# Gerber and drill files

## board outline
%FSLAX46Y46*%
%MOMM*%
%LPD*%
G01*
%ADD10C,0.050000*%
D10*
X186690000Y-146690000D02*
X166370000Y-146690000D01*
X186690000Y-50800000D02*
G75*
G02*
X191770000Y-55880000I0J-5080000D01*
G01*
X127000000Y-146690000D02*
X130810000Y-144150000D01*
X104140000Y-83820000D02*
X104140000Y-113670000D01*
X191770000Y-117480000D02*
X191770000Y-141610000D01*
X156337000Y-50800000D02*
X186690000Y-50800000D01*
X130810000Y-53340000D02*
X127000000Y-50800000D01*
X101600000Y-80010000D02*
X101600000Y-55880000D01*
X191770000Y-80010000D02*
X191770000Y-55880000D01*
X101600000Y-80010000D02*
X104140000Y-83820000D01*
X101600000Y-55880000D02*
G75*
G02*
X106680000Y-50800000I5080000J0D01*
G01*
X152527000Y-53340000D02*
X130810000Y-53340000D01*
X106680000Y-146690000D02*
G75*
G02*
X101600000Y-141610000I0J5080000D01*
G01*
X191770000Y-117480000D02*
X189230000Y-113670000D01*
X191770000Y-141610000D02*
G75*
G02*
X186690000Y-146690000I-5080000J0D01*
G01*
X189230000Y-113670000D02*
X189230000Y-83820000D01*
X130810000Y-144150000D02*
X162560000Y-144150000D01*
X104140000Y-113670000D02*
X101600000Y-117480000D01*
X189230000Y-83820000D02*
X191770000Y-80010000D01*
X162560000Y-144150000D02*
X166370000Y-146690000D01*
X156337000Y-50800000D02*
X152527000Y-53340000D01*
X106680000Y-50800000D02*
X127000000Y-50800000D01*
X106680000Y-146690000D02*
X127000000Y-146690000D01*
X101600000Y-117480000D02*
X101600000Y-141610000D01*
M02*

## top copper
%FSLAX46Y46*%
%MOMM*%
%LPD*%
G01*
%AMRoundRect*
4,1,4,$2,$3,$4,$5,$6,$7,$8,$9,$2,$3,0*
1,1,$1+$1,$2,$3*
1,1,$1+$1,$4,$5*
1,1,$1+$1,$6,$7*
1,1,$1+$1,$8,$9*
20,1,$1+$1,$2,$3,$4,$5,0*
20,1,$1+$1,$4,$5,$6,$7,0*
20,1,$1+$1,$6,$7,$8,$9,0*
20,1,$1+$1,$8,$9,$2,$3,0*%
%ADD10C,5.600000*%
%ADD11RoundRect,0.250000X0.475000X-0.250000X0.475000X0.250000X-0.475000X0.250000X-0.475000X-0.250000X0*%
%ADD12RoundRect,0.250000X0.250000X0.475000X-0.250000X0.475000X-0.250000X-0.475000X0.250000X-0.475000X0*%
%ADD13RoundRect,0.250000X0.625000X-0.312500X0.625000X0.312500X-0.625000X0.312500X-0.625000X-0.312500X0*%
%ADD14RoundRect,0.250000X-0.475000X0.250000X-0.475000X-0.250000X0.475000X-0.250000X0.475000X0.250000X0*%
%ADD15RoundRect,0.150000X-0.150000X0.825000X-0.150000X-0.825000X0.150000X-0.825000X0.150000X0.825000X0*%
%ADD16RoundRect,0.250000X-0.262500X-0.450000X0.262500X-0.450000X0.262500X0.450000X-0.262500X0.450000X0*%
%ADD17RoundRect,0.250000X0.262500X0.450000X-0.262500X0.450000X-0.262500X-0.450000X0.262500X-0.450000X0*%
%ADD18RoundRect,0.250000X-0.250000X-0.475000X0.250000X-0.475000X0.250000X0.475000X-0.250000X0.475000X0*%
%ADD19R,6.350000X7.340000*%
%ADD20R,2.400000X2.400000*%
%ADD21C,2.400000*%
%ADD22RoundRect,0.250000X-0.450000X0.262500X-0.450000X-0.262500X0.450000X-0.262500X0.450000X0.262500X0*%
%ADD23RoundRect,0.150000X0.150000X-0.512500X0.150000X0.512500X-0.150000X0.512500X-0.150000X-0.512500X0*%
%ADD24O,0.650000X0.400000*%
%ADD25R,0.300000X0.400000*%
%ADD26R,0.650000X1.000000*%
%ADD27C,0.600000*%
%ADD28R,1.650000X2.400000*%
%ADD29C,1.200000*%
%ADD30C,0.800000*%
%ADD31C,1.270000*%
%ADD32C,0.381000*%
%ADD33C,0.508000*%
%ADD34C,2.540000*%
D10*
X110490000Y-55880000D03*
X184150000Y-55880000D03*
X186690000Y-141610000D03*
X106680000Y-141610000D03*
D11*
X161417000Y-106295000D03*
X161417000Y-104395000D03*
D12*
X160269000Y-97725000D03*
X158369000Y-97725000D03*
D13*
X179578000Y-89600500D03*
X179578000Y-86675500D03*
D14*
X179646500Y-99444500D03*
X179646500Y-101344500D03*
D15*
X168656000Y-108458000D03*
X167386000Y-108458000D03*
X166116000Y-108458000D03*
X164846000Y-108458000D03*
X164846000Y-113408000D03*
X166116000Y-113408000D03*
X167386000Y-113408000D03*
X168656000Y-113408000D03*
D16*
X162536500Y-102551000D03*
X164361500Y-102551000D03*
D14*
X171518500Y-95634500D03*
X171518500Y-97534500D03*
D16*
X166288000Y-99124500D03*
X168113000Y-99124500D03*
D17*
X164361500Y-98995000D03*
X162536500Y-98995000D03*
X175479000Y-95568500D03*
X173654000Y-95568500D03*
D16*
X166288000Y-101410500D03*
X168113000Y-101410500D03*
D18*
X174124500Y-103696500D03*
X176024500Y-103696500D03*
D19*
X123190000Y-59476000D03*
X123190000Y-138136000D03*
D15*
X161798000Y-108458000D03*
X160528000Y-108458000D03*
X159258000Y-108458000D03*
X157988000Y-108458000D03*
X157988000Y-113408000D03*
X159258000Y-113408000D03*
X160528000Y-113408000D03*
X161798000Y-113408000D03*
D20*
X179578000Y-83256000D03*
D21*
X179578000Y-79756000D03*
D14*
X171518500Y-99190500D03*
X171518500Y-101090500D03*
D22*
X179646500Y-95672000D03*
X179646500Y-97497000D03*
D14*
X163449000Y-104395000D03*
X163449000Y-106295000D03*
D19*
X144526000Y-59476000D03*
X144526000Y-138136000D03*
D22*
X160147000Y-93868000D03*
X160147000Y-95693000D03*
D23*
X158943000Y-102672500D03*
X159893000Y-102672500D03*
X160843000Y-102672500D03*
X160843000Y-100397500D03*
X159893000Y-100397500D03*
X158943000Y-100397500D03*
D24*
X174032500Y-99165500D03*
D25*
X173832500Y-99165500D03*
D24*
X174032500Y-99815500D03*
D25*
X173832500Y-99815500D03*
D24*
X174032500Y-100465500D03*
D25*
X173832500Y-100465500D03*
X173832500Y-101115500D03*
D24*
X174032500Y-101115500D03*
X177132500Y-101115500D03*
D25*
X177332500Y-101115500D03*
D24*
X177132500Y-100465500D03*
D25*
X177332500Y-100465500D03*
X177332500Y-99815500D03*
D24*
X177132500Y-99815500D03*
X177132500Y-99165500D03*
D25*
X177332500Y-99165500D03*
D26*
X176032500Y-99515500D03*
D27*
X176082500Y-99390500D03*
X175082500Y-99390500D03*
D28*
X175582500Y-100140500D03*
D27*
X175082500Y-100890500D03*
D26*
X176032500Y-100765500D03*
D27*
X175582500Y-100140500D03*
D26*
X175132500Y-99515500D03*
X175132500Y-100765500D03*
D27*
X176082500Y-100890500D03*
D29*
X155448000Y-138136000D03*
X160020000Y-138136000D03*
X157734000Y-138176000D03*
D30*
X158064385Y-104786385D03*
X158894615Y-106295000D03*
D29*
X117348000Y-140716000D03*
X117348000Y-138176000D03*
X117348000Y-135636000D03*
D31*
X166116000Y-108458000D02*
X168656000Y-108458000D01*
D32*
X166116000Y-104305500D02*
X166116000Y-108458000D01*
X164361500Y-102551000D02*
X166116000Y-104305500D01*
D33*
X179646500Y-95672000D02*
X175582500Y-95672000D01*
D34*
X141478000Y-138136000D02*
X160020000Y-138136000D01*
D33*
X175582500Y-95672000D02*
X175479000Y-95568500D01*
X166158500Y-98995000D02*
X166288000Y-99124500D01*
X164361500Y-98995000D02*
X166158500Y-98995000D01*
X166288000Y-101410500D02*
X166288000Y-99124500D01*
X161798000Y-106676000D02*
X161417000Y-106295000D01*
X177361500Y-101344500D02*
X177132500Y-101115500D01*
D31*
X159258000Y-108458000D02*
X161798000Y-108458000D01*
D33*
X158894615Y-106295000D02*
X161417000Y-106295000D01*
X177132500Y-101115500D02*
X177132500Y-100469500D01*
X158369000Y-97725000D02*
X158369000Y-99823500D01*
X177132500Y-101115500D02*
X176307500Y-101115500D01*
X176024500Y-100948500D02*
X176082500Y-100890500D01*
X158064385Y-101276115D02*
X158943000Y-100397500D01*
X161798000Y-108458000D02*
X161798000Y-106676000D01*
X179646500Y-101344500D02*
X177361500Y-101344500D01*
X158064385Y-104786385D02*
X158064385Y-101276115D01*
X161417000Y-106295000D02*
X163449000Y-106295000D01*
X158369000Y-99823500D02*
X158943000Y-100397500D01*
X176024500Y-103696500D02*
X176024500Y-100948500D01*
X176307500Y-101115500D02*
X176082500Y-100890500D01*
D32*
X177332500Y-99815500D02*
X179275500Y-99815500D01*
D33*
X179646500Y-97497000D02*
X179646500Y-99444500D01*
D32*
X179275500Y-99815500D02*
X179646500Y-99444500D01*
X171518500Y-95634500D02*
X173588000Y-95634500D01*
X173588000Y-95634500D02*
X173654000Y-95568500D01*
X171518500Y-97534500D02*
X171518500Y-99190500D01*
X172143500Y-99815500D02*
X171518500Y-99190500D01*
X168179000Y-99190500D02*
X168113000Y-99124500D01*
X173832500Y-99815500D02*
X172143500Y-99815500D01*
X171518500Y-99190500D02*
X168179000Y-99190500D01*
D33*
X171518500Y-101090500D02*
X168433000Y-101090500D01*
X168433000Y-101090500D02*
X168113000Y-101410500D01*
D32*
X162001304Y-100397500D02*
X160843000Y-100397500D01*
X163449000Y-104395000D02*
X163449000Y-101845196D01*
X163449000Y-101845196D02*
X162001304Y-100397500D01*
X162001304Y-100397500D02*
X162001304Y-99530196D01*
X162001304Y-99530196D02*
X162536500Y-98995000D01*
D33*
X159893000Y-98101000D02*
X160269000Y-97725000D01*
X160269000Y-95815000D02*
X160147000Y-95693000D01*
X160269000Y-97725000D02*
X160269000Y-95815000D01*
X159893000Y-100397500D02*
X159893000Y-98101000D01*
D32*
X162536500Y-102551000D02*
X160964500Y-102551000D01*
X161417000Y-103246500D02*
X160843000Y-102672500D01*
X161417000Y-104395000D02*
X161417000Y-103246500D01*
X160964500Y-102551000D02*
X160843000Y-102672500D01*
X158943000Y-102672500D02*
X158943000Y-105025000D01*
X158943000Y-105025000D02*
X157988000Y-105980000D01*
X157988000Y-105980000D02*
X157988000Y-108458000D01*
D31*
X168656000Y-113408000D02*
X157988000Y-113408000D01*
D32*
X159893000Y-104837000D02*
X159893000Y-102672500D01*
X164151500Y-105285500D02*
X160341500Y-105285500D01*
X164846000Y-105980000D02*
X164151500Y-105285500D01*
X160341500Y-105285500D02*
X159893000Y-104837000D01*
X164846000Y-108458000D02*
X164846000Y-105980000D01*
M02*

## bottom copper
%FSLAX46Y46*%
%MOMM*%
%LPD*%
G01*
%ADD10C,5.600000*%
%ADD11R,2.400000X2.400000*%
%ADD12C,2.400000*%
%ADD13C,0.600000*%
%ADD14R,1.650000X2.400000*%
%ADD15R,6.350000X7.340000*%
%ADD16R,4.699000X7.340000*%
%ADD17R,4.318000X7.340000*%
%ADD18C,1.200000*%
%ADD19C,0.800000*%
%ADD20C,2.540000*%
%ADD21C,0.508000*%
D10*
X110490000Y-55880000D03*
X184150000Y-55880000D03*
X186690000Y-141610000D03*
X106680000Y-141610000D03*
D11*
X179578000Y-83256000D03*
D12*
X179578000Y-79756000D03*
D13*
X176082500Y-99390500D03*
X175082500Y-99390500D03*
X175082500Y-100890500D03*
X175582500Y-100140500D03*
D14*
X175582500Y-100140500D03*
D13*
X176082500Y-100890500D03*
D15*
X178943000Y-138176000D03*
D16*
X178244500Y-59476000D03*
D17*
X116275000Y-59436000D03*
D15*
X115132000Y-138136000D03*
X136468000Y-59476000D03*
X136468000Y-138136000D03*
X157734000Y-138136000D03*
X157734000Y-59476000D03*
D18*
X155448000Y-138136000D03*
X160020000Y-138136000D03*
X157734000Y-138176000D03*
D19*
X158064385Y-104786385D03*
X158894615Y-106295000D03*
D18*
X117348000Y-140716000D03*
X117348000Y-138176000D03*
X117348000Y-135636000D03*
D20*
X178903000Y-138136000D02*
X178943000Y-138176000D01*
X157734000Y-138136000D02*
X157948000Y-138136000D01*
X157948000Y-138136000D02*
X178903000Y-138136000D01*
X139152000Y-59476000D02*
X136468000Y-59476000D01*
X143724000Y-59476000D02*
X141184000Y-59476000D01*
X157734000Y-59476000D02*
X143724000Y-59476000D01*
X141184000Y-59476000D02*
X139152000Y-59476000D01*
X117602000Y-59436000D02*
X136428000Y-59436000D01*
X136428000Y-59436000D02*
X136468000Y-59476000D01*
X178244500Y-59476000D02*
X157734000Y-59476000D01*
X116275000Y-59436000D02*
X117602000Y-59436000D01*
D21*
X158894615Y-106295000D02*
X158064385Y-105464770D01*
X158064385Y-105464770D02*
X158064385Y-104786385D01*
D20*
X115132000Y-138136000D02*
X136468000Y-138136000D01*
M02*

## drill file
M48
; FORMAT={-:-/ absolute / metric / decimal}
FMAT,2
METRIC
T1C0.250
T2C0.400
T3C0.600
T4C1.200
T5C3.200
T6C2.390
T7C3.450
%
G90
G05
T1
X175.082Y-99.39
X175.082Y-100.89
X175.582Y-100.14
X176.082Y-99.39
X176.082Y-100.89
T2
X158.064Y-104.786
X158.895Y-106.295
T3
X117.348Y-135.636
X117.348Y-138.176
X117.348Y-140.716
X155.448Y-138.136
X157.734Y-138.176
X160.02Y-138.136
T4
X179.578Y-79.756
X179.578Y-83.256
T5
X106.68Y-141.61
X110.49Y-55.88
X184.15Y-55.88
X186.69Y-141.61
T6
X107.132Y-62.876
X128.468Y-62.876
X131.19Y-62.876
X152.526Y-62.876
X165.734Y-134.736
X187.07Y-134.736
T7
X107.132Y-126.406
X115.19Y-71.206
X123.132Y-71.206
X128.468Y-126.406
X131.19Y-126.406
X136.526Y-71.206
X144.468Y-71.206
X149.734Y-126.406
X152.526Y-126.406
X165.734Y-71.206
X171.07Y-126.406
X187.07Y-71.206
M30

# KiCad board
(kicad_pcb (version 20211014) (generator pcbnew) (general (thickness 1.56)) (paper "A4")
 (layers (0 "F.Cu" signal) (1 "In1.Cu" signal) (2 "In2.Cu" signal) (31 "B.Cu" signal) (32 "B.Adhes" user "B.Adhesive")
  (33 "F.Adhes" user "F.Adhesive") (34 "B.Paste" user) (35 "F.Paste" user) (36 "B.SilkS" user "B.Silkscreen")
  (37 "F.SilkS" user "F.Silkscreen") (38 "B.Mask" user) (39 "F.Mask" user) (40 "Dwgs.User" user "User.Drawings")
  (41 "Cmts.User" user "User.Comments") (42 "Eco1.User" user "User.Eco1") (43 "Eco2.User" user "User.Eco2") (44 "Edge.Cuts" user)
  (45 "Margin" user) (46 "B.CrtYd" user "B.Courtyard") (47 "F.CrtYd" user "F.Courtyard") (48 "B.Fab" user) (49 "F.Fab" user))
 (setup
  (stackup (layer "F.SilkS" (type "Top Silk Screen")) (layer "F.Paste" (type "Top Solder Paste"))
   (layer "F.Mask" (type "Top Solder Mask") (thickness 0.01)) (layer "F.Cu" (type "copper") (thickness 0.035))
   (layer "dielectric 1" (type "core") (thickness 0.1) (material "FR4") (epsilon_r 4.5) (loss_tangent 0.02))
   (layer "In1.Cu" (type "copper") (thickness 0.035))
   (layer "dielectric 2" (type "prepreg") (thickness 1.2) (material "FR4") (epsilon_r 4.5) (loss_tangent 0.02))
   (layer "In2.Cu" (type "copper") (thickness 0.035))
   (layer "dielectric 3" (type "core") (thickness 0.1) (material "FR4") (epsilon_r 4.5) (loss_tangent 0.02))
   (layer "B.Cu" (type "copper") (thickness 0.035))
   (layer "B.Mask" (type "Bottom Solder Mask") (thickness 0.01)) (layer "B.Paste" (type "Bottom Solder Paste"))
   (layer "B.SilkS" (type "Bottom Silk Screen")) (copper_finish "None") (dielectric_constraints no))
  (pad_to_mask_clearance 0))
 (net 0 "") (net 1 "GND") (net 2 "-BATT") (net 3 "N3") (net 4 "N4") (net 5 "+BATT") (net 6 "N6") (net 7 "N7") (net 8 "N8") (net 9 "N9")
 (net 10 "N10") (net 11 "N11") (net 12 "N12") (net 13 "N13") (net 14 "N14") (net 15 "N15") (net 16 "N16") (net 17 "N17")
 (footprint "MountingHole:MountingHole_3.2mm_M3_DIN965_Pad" (layer "F.Cu") (at 110.49 55.88)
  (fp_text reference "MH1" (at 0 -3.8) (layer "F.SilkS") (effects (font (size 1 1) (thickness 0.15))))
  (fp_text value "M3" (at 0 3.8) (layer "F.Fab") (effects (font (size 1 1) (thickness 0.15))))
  (pad "1" thru_hole circle (at 0 0) (size 5.6 5.6) (drill 3.2) (layers *.Cu *.Mask) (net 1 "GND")))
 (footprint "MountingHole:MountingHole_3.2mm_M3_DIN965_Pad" (layer "F.Cu") (at 184.15 55.88)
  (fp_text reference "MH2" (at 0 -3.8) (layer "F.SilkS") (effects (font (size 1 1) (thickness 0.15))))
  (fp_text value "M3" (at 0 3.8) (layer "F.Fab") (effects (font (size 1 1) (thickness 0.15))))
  (pad "1" thru_hole circle (at 0 0) (size 5.6 5.6) (drill 3.2) (layers *.Cu *.Mask) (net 1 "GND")))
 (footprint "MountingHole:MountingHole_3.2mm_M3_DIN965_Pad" (layer "F.Cu") (at 186.69 141.61)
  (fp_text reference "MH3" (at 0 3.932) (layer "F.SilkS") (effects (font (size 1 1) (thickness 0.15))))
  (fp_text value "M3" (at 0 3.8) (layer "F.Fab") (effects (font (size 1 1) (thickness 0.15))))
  (pad "1" thru_hole circle (at 0 0) (size 5.6 5.6) (drill 3.2) (layers *.Cu *.Mask) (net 1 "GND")))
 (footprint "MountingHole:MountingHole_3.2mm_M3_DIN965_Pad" (layer "F.Cu") (at 106.68 141.61)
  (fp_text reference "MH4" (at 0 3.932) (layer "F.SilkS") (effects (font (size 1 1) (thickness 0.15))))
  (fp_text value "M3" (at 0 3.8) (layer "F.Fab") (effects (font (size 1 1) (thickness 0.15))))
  (pad "1" thru_hole circle (at 0 0) (size 5.6 5.6) (drill 3.2) (layers *.Cu *.Mask) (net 1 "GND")))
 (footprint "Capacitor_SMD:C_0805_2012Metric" (layer "F.Cu") (at 161.417 105.345 90)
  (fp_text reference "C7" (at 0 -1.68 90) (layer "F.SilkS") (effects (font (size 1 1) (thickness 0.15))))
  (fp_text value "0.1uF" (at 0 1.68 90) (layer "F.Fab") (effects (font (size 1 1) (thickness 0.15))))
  (pad "1" smd roundrect (at -0.95 0 90) (size 1 1.45) (layers "F.Cu" "F.Paste" "F.Mask") (roundrect_rratio 0.25) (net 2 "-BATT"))
  (pad "2" smd roundrect (at 0.95 0 90) (size 1 1.45) (layers "F.Cu" "F.Paste" "F.Mask") (roundrect_rratio 0.25) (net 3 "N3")))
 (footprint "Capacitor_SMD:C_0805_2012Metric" (layer "F.Cu") (at 159.319 97.725 180)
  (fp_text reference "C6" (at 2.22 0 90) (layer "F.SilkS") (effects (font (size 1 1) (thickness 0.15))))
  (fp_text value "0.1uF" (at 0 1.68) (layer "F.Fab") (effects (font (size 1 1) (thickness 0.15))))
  (pad "1" smd roundrect (at -0.95 0 180) (size 1 1.45) (layers "F.Cu" "F.Paste" "F.Mask") (roundrect_rratio 0.25) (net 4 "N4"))
  (pad "2" smd roundrect (at 0.95 0 180) (size 1 1.45) (layers "F.Cu" "F.Paste" "F.Mask") (roundrect_rratio 0.25) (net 2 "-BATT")))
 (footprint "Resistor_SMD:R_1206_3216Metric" (layer "F.Cu") (at 179.578 88.138 90)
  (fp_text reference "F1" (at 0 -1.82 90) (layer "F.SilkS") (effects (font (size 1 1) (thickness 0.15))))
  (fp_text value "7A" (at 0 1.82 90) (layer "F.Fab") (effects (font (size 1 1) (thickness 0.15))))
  (pad "1" smd roundrect (at -1.4625 0 90) (size 1.125 1.75) (layers "F.Cu" "F.Paste" "F.Mask") (roundrect_rratio 0.222222) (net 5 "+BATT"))
  (pad "2" smd roundrect (at 1.4625 0 90) (size 1.125 1.75) (layers "F.Cu" "F.Paste" "F.Mask") (roundrect_rratio 0.222222) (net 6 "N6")))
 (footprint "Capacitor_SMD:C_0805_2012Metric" (layer "F.Cu") (at 179.6465 100.3945 -90)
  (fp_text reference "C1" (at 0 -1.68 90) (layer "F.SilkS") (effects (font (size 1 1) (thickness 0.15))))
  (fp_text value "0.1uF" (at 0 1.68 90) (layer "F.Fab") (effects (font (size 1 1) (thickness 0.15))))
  (pad "1" smd roundrect (at -0.95 0 270) (size 1 1.45) (layers "F.Cu" "F.Paste" "F.Mask") (roundrect_rratio 0.25) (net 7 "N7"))
  (pad "2" smd roundrect (at 0.95 0 270) (size 1 1.45) (layers "F.Cu" "F.Paste" "F.Mask") (roundrect_rratio 0.25) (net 2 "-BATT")))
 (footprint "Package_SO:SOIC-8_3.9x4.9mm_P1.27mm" (layer "F.Cu") (at 166.751 110.933 -90)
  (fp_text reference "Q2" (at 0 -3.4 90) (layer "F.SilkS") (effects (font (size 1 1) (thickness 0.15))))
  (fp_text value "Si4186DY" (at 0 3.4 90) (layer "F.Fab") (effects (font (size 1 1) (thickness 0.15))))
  (pad "1" smd roundrect (at -2.475 -1.905 270) (size 1.95 0.6) (layers "F.Cu" "F.Paste" "F.Mask") (roundrect_rratio 0.25) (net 1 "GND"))
  (pad "2" smd roundrect (at -2.475 -0.635 270) (size 1.95 0.6) (layers "F.Cu" "F.Paste" "F.Mask") (roundrect_rratio 0.25) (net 1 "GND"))
  (pad "3" smd roundrect (at -2.475 0.635 270) (size 1.95 0.6) (layers "F.Cu" "F.Paste" "F.Mask") (roundrect_rratio 0.25) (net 1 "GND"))
  (pad "4" smd roundrect (at -2.475 1.905 270) (size 1.95 0.6) (layers "F.Cu" "F.Paste" "F.Mask") (roundrect_rratio 0.25) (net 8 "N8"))
  (pad "5" smd roundrect (at 2.475 1.905 270) (size 1.95 0.6) (layers "F.Cu" "F.Paste" "F.Mask") (roundrect_rratio 0.25) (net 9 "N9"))
  (pad "6" smd roundrect (at 2.475 0.635 270) (size 1.95 0.6) (layers "F.Cu" "F.Paste" "F.Mask") (roundrect_rratio 0.25) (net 9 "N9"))
  (pad "7" smd roundrect (at 2.475 -0.635 270) (size 1.95 0.6) (layers "F.Cu" "F.Paste" "F.Mask") (roundrect_rratio 0.25) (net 9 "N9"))
  (pad "8" smd roundrect (at 2.475 -1.905 270) (size 1.95 0.6) (layers "F.Cu" "F.Paste" "F.Mask") (roundrect_rratio 0.25) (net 9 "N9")))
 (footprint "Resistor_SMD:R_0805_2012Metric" (layer "F.Cu") (at 163.449 102.551)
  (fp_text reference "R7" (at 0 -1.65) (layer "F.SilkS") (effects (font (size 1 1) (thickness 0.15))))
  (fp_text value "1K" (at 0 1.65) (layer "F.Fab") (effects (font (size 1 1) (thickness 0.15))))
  (pad "1" smd roundrect (at -0.9125 0) (size 1.025 1.4) (layers "F.Cu" "F.Paste" "F.Mask") (roundrect_rratio 0.243902) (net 3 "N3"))
  (pad "2" smd roundrect (at 0.9125 0) (size 1.025 1.4) (layers "F.Cu" "F.Paste" "F.Mask") (roundrect_rratio 0.243902) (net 1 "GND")))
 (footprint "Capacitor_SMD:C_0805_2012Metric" (layer "F.Cu") (at 171.5185 96.5845 -90)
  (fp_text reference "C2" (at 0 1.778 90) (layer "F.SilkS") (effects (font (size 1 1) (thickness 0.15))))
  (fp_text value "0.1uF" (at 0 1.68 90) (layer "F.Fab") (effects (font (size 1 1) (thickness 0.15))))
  (pad "1" smd roundrect (at -0.95 0 270) (size 1 1.45) (layers "F.Cu" "F.Paste" "F.Mask") (roundrect_rratio 0.25) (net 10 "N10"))
  (pad "2" smd roundrect (at 0.95 0 270) (size 1 1.45) (layers "F.Cu" "F.Paste" "F.Mask") (roundrect_rratio 0.25) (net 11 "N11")))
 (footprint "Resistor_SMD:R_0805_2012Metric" (layer "F.Cu") (at 167.2005 99.1245)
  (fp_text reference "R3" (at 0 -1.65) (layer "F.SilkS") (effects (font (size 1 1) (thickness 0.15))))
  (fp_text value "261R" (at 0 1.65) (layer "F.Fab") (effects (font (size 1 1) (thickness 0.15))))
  (pad "1" smd roundrect (at -0.9125 0) (size 1.025 1.4) (layers "F.Cu" "F.Paste" "F.Mask") (roundrect_rratio 0.243902) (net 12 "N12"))
  (pad "2" smd roundrect (at 0.9125 0) (size 1.025 1.4) (layers "F.Cu" "F.Paste" "F.Mask") (roundrect_rratio 0.243902) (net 11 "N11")))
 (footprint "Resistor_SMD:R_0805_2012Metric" (layer "F.Cu") (at 163.449 98.995 180)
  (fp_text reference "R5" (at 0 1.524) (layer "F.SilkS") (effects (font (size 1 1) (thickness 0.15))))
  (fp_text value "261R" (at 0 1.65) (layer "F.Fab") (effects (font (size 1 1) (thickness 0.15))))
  (pad "1" smd roundrect (at -0.9125 0 180) (size 1.025 1.4) (layers "F.Cu" "F.Paste" "F.Mask") (roundrect_rratio 0.243902) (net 12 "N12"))
  (pad "2" smd roundrect (at 0.9125 0 180) (size 1.025 1.4) (layers "F.Cu" "F.Paste" "F.Mask") (roundrect_rratio 0.243902) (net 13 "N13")))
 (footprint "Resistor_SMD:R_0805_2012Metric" (layer "F.Cu") (at 174.5665 95.5685 180)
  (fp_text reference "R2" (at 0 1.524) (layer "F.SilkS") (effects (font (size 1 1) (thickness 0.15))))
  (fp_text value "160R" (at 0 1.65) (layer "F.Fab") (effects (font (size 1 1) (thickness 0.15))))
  (pad "1" smd roundrect (at -0.9125 0 180) (size 1.025 1.4) (layers "F.Cu" "F.Paste" "F.Mask") (roundrect_rratio 0.243902) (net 5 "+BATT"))
  (pad "2" smd roundrect (at 0.9125 0 180) (size 1.025 1.4) (layers "F.Cu" "F.Paste" "F.Mask") (roundrect_rratio 0.243902) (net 10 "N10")))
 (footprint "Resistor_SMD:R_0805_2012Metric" (layer "F.Cu") (at 167.2005 101.4105)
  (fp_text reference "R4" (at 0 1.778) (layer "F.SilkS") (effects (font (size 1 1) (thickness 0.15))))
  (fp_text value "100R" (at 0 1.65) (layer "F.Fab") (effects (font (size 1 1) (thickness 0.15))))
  (pad "1" smd roundrect (at -0.9125 0) (size 1.025 1.4) (layers "F.Cu" "F.Paste" "F.Mask") (roundrect_rratio 0.243902) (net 12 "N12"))
  (pad "2" smd roundrect (at 0.9125 0) (size 1.025 1.4) (layers "F.Cu" "F.Paste" "F.Mask") (roundrect_rratio 0.243902) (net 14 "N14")))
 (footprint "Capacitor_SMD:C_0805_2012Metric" (layer "F.Cu") (at 175.0745 103.6965)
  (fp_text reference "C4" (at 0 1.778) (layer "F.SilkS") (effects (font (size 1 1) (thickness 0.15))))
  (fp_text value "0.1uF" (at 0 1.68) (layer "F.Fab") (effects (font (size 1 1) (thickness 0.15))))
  (pad "1" smd roundrect (at -0.95 0) (size 1 1.45) (layers "F.Cu" "F.Paste" "F.Mask") (roundrect_rratio 0.25) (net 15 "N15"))
  (pad "2" smd roundrect (at 0.95 0) (size 1 1.45) (layers "F.Cu" "F.Paste" "F.Mask") (roundrect_rratio 0.25) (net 2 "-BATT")))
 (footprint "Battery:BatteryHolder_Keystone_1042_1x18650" (layer "F.Cu") (at 123.19 98.806 -90)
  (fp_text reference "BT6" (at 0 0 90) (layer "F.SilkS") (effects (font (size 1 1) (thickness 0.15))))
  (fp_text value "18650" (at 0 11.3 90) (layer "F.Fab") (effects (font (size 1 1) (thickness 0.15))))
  (pad "" np_thru_hole circle (at -35.93 -8 270) (size 2.39 2.39) (drill 2.39) (layers *.Cu *.Mask))
  (pad "" np_thru_hole circle (at 27.6 -8 270) (size 3.45 3.45) (drill 3.45) (layers *.Cu *.Mask))
  (pad "" np_thru_hole circle (at -27.6 8 270) (size 3.45 3.45) (drill 3.45) (layers *.Cu *.Mask))
  (pad "1" smd rect (at -39.33 0 270) (size 7.34 6.35) (layers "F.Cu" "F.Paste" "F.Mask") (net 12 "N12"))
  (pad "2" smd rect (at 39.33 0 270) (size 7.34 6.35) (layers "F.Cu" "F.Paste" "F.Mask") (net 2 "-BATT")))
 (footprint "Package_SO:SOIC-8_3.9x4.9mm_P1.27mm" (layer "F.Cu") (at 159.893 110.933 -90)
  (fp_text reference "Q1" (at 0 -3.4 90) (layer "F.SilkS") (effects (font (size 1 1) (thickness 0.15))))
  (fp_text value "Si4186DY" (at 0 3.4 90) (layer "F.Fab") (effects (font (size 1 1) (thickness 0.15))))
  (pad "1" smd roundrect (at -2.475 -1.905 270) (size 1.95 0.6) (layers "F.Cu" "F.Paste" "F.Mask") (roundrect_rratio 0.25) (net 2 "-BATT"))
  (pad "2" smd roundrect (at -2.475 -0.635 270) (size 1.95 0.6) (layers "F.Cu" "F.Paste" "F.Mask") (roundrect_rratio 0.25) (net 2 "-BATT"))
  (pad "3" smd roundrect (at -2.475 0.635 270) (size 1.95 0.6) (layers "F.Cu" "F.Paste" "F.Mask") (roundrect_rratio 0.25) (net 2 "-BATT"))
  (pad "4" smd roundrect (at -2.475 1.905 270) (size 1.95 0.6) (layers "F.Cu" "F.Paste" "F.Mask") (roundrect_rratio 0.25) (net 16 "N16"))
  (pad "5" smd roundrect (at 2.475 1.905 270) (size 1.95 0.6) (layers "F.Cu" "F.Paste" "F.Mask") (roundrect_rratio 0.25) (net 9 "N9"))
  (pad "6" smd roundrect (at 2.475 0.635 270) (size 1.95 0.6) (layers "F.Cu" "F.Paste" "F.Mask") (roundrect_rratio 0.25) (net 9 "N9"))
  (pad "7" smd roundrect (at 2.475 -0.635 270) (size 1.95 0.6) (layers "F.Cu" "F.Paste" "F.Mask") (roundrect_rratio 0.25) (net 9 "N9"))
  (pad "8" smd roundrect (at 2.475 -1.905 270) (size 1.95 0.6) (layers "F.Cu" "F.Paste" "F.Mask") (roundrect_rratio 0.25) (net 9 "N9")))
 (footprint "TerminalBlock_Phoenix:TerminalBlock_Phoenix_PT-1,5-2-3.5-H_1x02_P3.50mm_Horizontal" (layer "F.Cu") (at 179.578 83.256 90)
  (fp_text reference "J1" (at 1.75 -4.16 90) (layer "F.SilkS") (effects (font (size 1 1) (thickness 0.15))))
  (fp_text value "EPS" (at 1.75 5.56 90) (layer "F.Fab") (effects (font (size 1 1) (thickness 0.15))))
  (pad "1" thru_hole rect (at 0 0 90) (size 2.4 2.4) (drill 1.2) (layers *.Cu *.Mask) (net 6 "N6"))
  (pad "2" thru_hole circle (at 3.5 0 90) (size 2.4 2.4) (drill 1.2) (layers *.Cu *.Mask) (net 1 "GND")))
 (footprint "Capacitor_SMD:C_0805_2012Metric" (layer "F.Cu") (at 171.5185 100.1405 -90)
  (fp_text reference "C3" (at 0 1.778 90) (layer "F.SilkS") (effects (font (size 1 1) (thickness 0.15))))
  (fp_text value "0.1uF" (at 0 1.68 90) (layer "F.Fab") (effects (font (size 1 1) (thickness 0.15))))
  (pad "1" smd roundrect (at -0.95 0 270) (size 1 1.45) (layers "F.Cu" "F.Paste" "F.Mask") (roundrect_rratio 0.25) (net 11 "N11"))
  (pad "2" smd roundrect (at 0.95 0 270) (size 1 1.45) (layers "F.Cu" "F.Paste" "F.Mask") (roundrect_rratio 0.25) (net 14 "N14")))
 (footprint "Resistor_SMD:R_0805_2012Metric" (layer "F.Cu") (at 179.6465 96.5845 -90)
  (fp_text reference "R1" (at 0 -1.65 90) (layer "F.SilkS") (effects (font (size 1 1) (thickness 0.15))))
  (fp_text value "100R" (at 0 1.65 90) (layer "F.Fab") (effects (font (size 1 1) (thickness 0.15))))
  (pad "1" smd roundrect (at -0.9125 0 270) (size 1.025 1.4) (layers "F.Cu" "F.Paste" "F.Mask") (roundrect_rratio 0.243902) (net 5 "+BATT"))
  (pad "2" smd roundrect (at 0.9125 0 270) (size 1.025 1.4) (layers "F.Cu" "F.Paste" "F.Mask") (roundrect_rratio 0.243902) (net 7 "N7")))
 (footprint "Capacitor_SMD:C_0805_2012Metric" (layer "F.Cu") (at 163.449 105.345 -90)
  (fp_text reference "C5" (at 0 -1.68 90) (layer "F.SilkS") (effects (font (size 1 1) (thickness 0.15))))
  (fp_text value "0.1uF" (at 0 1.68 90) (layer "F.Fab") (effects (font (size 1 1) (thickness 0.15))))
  (pad "1" smd roundrect (at -0.95 0 270) (size 1 1.45) (layers "F.Cu" "F.Paste" "F.Mask") (roundrect_rratio 0.25) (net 13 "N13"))
  (pad "2" smd roundrect (at 0.95 0 270) (size 1 1.45) (layers "F.Cu" "F.Paste" "F.Mask") (roundrect_rratio 0.25) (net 2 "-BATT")))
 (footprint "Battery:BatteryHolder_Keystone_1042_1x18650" (layer "F.Cu") (at 144.526 98.806 -90)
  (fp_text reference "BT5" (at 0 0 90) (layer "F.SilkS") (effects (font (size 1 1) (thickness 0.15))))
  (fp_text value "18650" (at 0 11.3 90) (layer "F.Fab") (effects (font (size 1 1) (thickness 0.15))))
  (pad "" np_thru_hole circle (at -27.6 8 270) (size 3.45 3.45) (drill 3.45) (layers *.Cu *.Mask))
  (pad "" np_thru_hole circle (at -35.93 -8 270) (size 2.39 2.39) (drill 2.39) (layers *.Cu *.Mask))
  (pad "" np_thru_hole circle (at 27.6 -8 270) (size 3.45 3.45) (drill 3.45) (layers *.Cu *.Mask))
  (pad "1" smd rect (at -39.33 0 270) (size 7.34 6.35) (layers "F.Cu" "F.Paste" "F.Mask") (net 5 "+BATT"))
  (pad "2" smd rect (at 39.33 0 270) (size 7.34 6.35) (layers "F.Cu" "F.Paste" "F.Mask") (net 12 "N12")))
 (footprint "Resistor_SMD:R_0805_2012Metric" (layer "F.Cu") (at 160.147 94.7805 -90)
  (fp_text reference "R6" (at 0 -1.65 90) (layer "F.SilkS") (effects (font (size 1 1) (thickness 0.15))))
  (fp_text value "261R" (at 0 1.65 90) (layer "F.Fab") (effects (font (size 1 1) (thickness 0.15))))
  (pad "1" smd roundrect (at -0.9125 0 270) (size 1.025 1.4) (layers "F.Cu" "F.Paste" "F.Mask") (roundrect_rratio 0.243902) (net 5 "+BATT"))
  (pad "2" smd roundrect (at 0.9125 0 270) (size 1.025 1.4) (layers "F.Cu" "F.Paste" "F.Mask") (roundrect_rratio 0.243902) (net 4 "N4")))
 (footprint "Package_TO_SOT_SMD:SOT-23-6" (layer "F.Cu") (at 159.893 101.535 90)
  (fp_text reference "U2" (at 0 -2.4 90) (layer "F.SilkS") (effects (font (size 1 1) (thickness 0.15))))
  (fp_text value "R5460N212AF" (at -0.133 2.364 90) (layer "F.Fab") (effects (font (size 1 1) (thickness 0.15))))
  (pad "1" smd roundrect (at -1.1375 -0.95 90) (size 1.325 0.6) (layers "F.Cu" "F.Paste" "F.Mask") (roundrect_rratio 0.25) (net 16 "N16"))
  (pad "2" smd roundrect (at -1.1375 0 90) (size 1.325 0.6) (layers "F.Cu" "F.Paste" "F.Mask") (roundrect_rratio 0.25) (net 8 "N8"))
  (pad "3" smd roundrect (at -1.1375 0.95 90) (size 1.325 0.6) (layers "F.Cu" "F.Paste" "F.Mask") (roundrect_rratio 0.25) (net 3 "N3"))
  (pad "4" smd roundrect (at 1.1375 0.95 90) (size 1.325 0.6) (layers "F.Cu" "F.Paste" "F.Mask") (roundrect_rratio 0.25) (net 13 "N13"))
  (pad "5" smd roundrect (at 1.1375 0 90) (size 1.325 0.6) (layers "F.Cu" "F.Paste" "F.Mask") (roundrect_rratio 0.25) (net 4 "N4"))
  (pad "6" smd roundrect (at 1.1375 -0.95 90) (size 1.325 0.6) (layers "F.Cu" "F.Paste" "F.Mask") (roundrect_rratio 0.25) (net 2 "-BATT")))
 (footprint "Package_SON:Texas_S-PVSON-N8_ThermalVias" (layer "F.Cu") (at 175.5825 100.1405)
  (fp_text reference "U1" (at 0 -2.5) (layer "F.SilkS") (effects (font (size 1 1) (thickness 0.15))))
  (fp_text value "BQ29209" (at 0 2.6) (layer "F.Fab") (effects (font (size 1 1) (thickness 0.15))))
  (pad "1" smd oval (at -1.55 -0.975) (size 0.65 0.4) (layers "F.Cu" "F.Paste" "F.Mask") (solder_paste_margin -0.05))
  (pad "1" smd rect (at -1.75 -0.975) (size 0.3 0.4) (layers "F.Cu" "F.Paste" "F.Mask") (solder_paste_margin -0.05))
  (pad "2" smd oval (at -1.55 -0.325) (size 0.65 0.4) (layers "F.Cu" "F.Paste" "F.Mask") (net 11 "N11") (solder_paste_margin -0.05))
  (pad "2" smd rect (at -1.75 -0.325) (size 0.3 0.4) (layers "F.Cu" "F.Paste" "F.Mask") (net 11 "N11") (solder_paste_margin -0.05))
  (pad "3" smd oval (at -1.55 0.325) (size 0.65 0.4) (layers "F.Cu" "F.Paste" "F.Mask") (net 14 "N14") (solder_paste_margin -0.05))
  (pad "3" smd rect (at -1.75 0.325) (size 0.3 0.4) (layers "F.Cu" "F.Paste" "F.Mask") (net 14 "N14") (solder_paste_margin -0.05))
  (pad "4" smd rect (at -1.75 0.975) (size 0.3 0.4) (layers "F.Cu" "F.Paste" "F.Mask") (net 15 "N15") (solder_paste_margin -0.05))
  (pad "4" smd oval (at -1.55 0.975) (size 0.65 0.4) (layers "F.Cu" "F.Paste" "F.Mask") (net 15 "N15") (solder_paste_margin -0.05))
  (pad "5" smd oval (at 1.55 0.975) (size 0.65 0.4) (layers "F.Cu" "F.Paste" "F.Mask") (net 2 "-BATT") (solder_paste_margin -0.05))
  (pad "5" smd rect (at 1.75 0.975) (size 0.3 0.4) (layers "F.Cu" "F.Paste" "F.Mask") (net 2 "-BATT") (solder_paste_margin -0.05))
  (pad "6" smd oval (at 1.55 0.325) (size 0.65 0.4) (layers "F.Cu" "F.Paste" "F.Mask") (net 2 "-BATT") (solder_paste_margin -0.05))
  (pad "6" smd rect (at 1.75 0.325) (size 0.3 0.4) (layers "F.Cu" "F.Paste" "F.Mask") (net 2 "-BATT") (solder_paste_margin -0.05))
  (pad "7" smd rect (at 1.75 -0.325) (size 0.3 0.4) (layers "F.Cu" "F.Paste" "F.Mask") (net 7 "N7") (solder_paste_margin -0.05))
  (pad "7" smd oval (at 1.55 -0.325) (size 0.65 0.4) (layers "F.Cu" "F.Paste" "F.Mask") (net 7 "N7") (solder_paste_margin -0.05))
  (pad "8" smd oval (at 1.55 -0.975) (size 0.65 0.4) (layers "F.Cu" "F.Paste" "F.Mask") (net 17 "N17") (solder_paste_margin -0.05))
  (pad "8" smd rect (at 1.75 -0.975) (size 0.3 0.4) (layers "F.Cu" "F.Paste" "F.Mask") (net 17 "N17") (solder_paste_margin -0.05))
  (pad "9" smd rect (at 0.45 -0.625) (size 0.65 1) (layers "F.Cu" "F.Paste" "F.Mask") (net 2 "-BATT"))
  (pad "9" thru_hole circle (at 0.5 -0.75) (size 0.6 0.6) (drill 0.25) (layers *.Cu) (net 2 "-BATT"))
  (pad "9" thru_hole circle (at -0.5 -0.75) (size 0.6 0.6) (drill 0.25) (layers *.Cu) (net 2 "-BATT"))
  (pad "9" smd rect (at 0 0) (size 1.65 2.4) (layers "F.Cu" "F.Mask") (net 2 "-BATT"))
  (pad "9" thru_hole circle (at -0.5 0.75) (size 0.6 0.6) (drill 0.25) (layers *.Cu) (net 2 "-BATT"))
  (pad "9" smd rect (at 0.45 0.625) (size 0.65 1) (layers "F.Cu" "F.Paste" "F.Mask") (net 2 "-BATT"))
  (pad "9" thru_hole circle (at 0 0) (size 0.6 0.6) (drill 0.25) (layers *.Cu) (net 2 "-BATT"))
  (pad "9" smd rect (at -0.45 -0.625) (size 0.65 1) (layers "F.Cu" "F.Paste" "F.Mask") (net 2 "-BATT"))
  (pad "9" smd rect (at -0.45 0.625) (size 0.65 1) (layers "F.Cu" "F.Paste" "F.Mask") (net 2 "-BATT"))
  (pad "9" smd rect (at 0 0) (size 1.65 2.4) (layers "B.Cu") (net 2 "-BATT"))
  (pad "9" thru_hole circle (at 0.5 0.75) (size 0.6 0.6) (drill 0.25) (layers *.Cu) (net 2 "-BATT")))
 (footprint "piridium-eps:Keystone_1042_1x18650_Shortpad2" (layer "B.Cu") (at 179.07 98.806 90)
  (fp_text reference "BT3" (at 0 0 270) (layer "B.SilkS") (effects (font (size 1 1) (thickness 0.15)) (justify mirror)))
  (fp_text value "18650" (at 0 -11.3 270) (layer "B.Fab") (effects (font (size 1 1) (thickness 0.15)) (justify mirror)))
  (pad "" np_thru_hole circle (at -35.93 8 90) (size 2.39 2.39) (drill 2.39) (layers *.Cu *.Mask))
  (pad "" np_thru_hole circle (at -27.6 -8 90) (size 3.45 3.45) (drill 3.45) (layers *.Cu *.Mask))
  (pad "" np_thru_hole circle (at 27.6 8 90) (size 3.45 3.45) (drill 3.45) (layers *.Cu *.Mask))
  (pad "1" smd rect (at -39.37 -0.127 90) (size 7.34 6.35) (layers "B.Cu" "B.Paste" "B.Mask") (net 5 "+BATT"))
  (pad "2" smd rect (at 39.33 -0.8255 90) (size 7.34 4.699) (layers "B.Cu" "B.Paste" "B.Mask") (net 12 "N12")))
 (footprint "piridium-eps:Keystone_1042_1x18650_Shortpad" (layer "B.Cu") (at 115.132 98.806 -90)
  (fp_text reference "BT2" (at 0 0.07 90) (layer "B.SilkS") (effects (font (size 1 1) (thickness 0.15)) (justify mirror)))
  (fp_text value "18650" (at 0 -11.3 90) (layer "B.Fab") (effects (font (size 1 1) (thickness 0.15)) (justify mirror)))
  (pad "" np_thru_hole circle (at -27.6 -8 270) (size 3.45 3.45) (drill 3.45) (layers *.Cu *.Mask))
  (pad "" np_thru_hole circle (at 27.6 8 270) (size 3.45 3.45) (drill 3.45) (layers *.Cu *.Mask))
  (pad "" np_thru_hole circle (at -35.93 8 270) (size 2.39 2.39) (drill 2.39) (layers *.Cu *.Mask))
  (pad "1" smd rect (at -39.37 -1.143 270) (size 7.34 4.318) (layers "B.Cu" "B.Paste" "B.Mask") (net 12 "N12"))
  (pad "2" smd rect (at 39.33 0 270) (size 7.34 6.35) (layers "B.Cu" "B.Paste" "B.Mask") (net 2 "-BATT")))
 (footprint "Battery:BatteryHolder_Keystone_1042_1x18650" (layer "B.Cu") (at 136.468 98.806 -90)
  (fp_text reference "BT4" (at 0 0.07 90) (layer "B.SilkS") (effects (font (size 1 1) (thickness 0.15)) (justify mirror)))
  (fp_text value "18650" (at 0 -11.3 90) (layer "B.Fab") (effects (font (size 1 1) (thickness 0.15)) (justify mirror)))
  (pad "" np_thru_hole circle (at -35.93 8 270) (size 2.39 2.39) (drill 2.39) (layers *.Cu *.Mask))
  (pad "" np_thru_hole circle (at 27.6 8 270) (size 3.45 3.45) (drill 3.45) (layers *.Cu *.Mask))
  (pad "" np_thru_hole circle (at -27.6 -8 270) (size 3.45 3.45) (drill 3.45) (layers *.Cu *.Mask))
  (pad "1" smd rect (at -39.33 0 270) (size 7.34 6.35) (layers "B.Cu" "B.Paste" "B.Mask") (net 12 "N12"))
  (pad "2" smd rect (at 39.33 0 270) (size 7.34 6.35) (layers "B.Cu" "B.Paste" "B.Mask") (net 2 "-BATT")))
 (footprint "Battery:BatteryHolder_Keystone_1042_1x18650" (layer "B.Cu") (at 157.734 98.806 90)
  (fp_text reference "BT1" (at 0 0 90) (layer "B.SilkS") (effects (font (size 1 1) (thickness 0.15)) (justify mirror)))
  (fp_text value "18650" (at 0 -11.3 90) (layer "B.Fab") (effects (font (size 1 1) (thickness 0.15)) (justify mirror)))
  (pad "" np_thru_hole circle (at -27.6 -8 90) (size 3.45 3.45) (drill 3.45) (layers *.Cu *.Mask))
  (pad "" np_thru_hole circle (at 27.6 8 90) (size 3.45 3.45) (drill 3.45) (layers *.Cu *.Mask))
  (pad "" np_thru_hole circle (at -35.93 8 90) (size 2.39 2.39) (drill 2.39) (layers *.Cu *.Mask))
  (pad "1" smd rect (at -39.33 0 90) (size 7.34 6.35) (layers "B.Cu" "B.Paste" "B.Mask") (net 5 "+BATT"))
  (pad "2" smd rect (at 39.33 0 90) (size 7.34 6.35) (layers "B.Cu" "B.Paste" "B.Mask") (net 12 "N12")))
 (gr_line (start 186.69 146.69) (end 166.37 146.69) (layer "Edge.Cuts") (width 0.05))
 (gr_arc (start 186.69 50.8) (mid 190.282102 52.287898) (end 191.77 55.88) (layer "Edge.Cuts") (width 0.05))
 (gr_line (start 127 146.69) (end 130.81 144.15) (layer "Edge.Cuts") (width 0.05))
 (gr_line (start 104.14 83.82) (end 104.14 113.67) (layer "Edge.Cuts") (width 0.05))
 (gr_line (start 191.77 117.48) (end 191.77 141.61) (layer "Edge.Cuts") (width 0.05))
 (gr_line (start 156.337 50.8) (end 186.69 50.8) (layer "Edge.Cuts") (width 0.05))
 (gr_line (start 130.81 53.34) (end 127 50.8) (layer "Edge.Cuts") (width 0.05))
 (gr_line (start 101.6 80.01) (end 101.6 55.88) (layer "Edge.Cuts") (width 0.05))
 (gr_line (start 191.77 80.01) (end 191.77 55.88) (layer "Edge.Cuts") (width 0.05))
 (gr_line (start 101.6 80.01) (end 104.14 83.82) (layer "Edge.Cuts") (width 0.05))
 (gr_arc (start 101.6 55.88) (mid 103.087898 52.287898) (end 106.68 50.8) (layer "Edge.Cuts") (width 0.05))
 (gr_line (start 152.527 53.34) (end 130.81 53.34) (layer "Edge.Cuts") (width 0.05))
 (gr_arc (start 106.68 146.69) (mid 103.087898 145.202102) (end 101.6 141.61) (layer "Edge.Cuts") (width 0.05))
 (gr_line (start 191.77 117.48) (end 189.23 113.67) (layer "Edge.Cuts") (width 0.05))
 (gr_arc (start 191.77 141.61) (mid 190.282102 145.202102) (end 186.69 146.69) (layer "Edge.Cuts") (width 0.05))
 (gr_line (start 189.23 113.67) (end 189.23 83.82) (layer "Edge.Cuts") (width 0.05))
 (gr_line (start 130.81 144.15) (end 162.56 144.15) (layer "Edge.Cuts") (width 0.05))
 (gr_line (start 104.14 113.67) (end 101.6 117.48) (layer "Edge.Cuts") (width 0.05))
 (gr_line (start 189.23 83.82) (end 191.77 80.01) (layer "Edge.Cuts") (width 0.05))
 (gr_line (start 162.56 144.15) (end 166.37 146.69) (layer "Edge.Cuts") (width 0.05))
 (gr_line (start 156.337 50.8) (end 152.527 53.34) (layer "Edge.Cuts") (width 0.05))
 (gr_line (start 106.68 50.8) (end 127 50.8) (layer "Edge.Cuts") (width 0.05))
 (gr_line (start 106.68 146.69) (end 127 146.69) (layer "Edge.Cuts") (width 0.05))
 (gr_line (start 101.6 117.48) (end 101.6 141.61) (layer "Edge.Cuts") (width 0.05))
 (segment (start 166.116 108.458) (end 168.656 108.458) (width 1.27) (layer "F.Cu") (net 1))
 (segment (start 166.116 104.3055) (end 166.116 108.458) (width 0.381) (layer "F.Cu") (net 1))
 (segment (start 164.3615 102.551) (end 166.116 104.3055) (width 0.381) (layer "F.Cu") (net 1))
 (segment (start 179.6465 95.672) (end 175.5825 95.672) (width 0.508) (layer "F.Cu") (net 5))
 (segment (start 141.478 138.136) (end 160.02 138.136) (width 2.54) (layer "F.Cu") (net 5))
 (segment (start 175.5825 95.672) (end 175.479 95.5685) (width 0.508) (layer "F.Cu") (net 5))
 (via (at 155.448 138.136) (size 1.2) (drill 0.6) (layers "F.Cu" "B.Cu") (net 5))
 (via (at 160.02 138.136) (size 1.2) (drill 0.6) (layers "F.Cu" "B.Cu") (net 5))
 (via (at 157.734 138.176) (size 1.2) (drill 0.6) (layers "F.Cu" "B.Cu") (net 5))
 (segment (start 178.903 138.136) (end 178.943 138.176) (width 2.54) (layer "B.Cu") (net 5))
 (segment (start 157.734 138.136) (end 157.948 138.136) (width 2.54) (layer "B.Cu") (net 5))
 (segment (start 157.948 138.136) (end 178.903 138.136) (width 2.54) (layer "B.Cu") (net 5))
 (segment (start 166.1585 98.995) (end 166.288 99.1245) (width 0.508) (layer "F.Cu") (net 12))
 (segment (start 164.3615 98.995) (end 166.1585 98.995) (width 0.508) (layer "F.Cu") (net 12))
 (segment (start 166.288 101.4105) (end 166.288 99.1245) (width 0.508) (layer "F.Cu") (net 12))
 (segment (start 139.152 59.476) (end 136.468 59.476) (width 2.54) (layer "B.Cu") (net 12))
 (segment (start 143.724 59.476) (end 141.184 59.476) (width 2.54) (layer "B.Cu") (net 12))
 (segment (start 157.734 59.476) (end 143.724 59.476) (width 2.54) (layer "B.Cu") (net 12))
 (segment (start 141.184 59.476) (end 139.152 59.476) (width 2.54) (layer "B.Cu") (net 12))
 (segment (start 117.602 59.436) (end 136.428 59.436) (width 2.54) (layer "B.Cu") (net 12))
 (segment (start 136.428 59.436) (end 136.468 59.476) (width 2.54) (layer "B.Cu") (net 12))
 (segment (start 178.2445 59.476) (end 157.734 59.476) (width 2.54) (layer "B.Cu") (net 12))
 (segment (start 116.275 59.436) (end 117.602 59.436) (width 2.54) (layer "B.Cu") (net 12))
 (segment (start 161.798 106.676) (end 161.417 106.295) (width 0.508) (layer "F.Cu") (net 2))
 (segment (start 177.3615 101.3445) (end 177.1325 101.1155) (width 0.508) (layer "F.Cu") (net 2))
 (segment (start 159.258 108.458) (end 161.798 108.458) (width 1.27) (layer "F.Cu") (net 2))
 (segment (start 158.894615 106.295) (end 161.417 106.295) (width 0.508) (layer "F.Cu") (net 2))
 (segment (start 177.1325 101.1155) (end 177.1325 100.4695) (width 0.508) (layer "F.Cu") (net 2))
 (segment (start 158.369 97.725) (end 158.369 99.8235) (width 0.508) (layer "F.Cu") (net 2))
 (segment (start 177.1325 101.1155) (end 176.3075 101.1155) (width 0.508) (layer "F.Cu") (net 2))
 (segment (start 176.0245 100.9485) (end 176.0825 100.8905) (width 0.508) (layer "F.Cu") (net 2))
 (segment (start 158.064385 101.276115) (end 158.943 100.3975) (width 0.508) (layer "F.Cu") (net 2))
 (segment (start 161.798 108.458) (end 161.798 106.676) (width 0.508) (layer "F.Cu") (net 2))
 (segment (start 179.6465 101.3445) (end 177.3615 101.3445) (width 0.508) (layer "F.Cu") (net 2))
 (segment (start 158.064385 104.786385) (end 158.064385 101.276115) (width 0.508) (layer "F.Cu") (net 2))
 (segment (start 161.417 106.295) (end 163.449 106.295) (width 0.508) (layer "F.Cu") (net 2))
 (segment (start 158.369 99.8235) (end 158.943 100.3975) (width 0.508) (layer "F.Cu") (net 2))
 (segment (start 176.0245 103.6965) (end 176.0245 100.9485) (width 0.508) (layer "F.Cu") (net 2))
 (segment (start 176.3075 101.1155) (end 176.0825 100.8905) (width 0.508) (layer "F.Cu") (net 2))
 (via (at 158.064385 104.786385) (size 0.8) (drill 0.4) (layers "F.Cu" "B.Cu") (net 2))
 (via (at 158.894615 106.295) (size 0.8) (drill 0.4) (layers "F.Cu" "B.Cu") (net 2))
 (via (at 117.348 140.716) (size 1.2) (drill 0.6) (layers "F.Cu" "B.Cu") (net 2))
 (via (at 117.348 138.176) (size 1.2) (drill 0.6) (layers "F.Cu" "B.Cu") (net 2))
 (via (at 117.348 135.636) (size 1.2) (drill 0.6) (layers "F.Cu" "B.Cu") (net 2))
 (segment (start 158.894615 106.295) (end 158.064385 105.46477) (width 0.508) (layer "B.Cu") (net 2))
 (segment (start 158.064385 105.46477) (end 158.064385 104.786385) (width 0.508) (layer "B.Cu") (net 2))
 (segment (start 115.132 138.136) (end 136.468 138.136) (width 2.54) (layer "B.Cu") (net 2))
 (segment (start 177.3325 99.8155) (end 179.2755 99.8155) (width 0.381) (layer "F.Cu") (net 7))
 (segment (start 179.6465 97.497) (end 179.6465 99.4445) (width 0.508) (layer "F.Cu") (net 7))
 (segment (start 179.2755 99.8155) (end 179.6465 99.4445) (width 0.381) (layer "F.Cu") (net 7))
 (segment (start 171.5185 95.6345) (end 173.588 95.6345) (width 0.381) (layer "F.Cu") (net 10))
 (segment (start 173.588 95.6345) (end 173.654 95.5685) (width 0.381) (layer "F.Cu") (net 10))
 (segment (start 171.5185 97.5345) (end 171.5185 99.1905) (width 0.381) (layer "F.Cu") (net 11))
 (segment (start 172.1435 99.8155) (end 171.5185 99.1905) (width 0.381) (layer "F.Cu") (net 11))
 (segment (start 168.179 99.1905) (end 168.113 99.1245) (width 0.381) (layer "F.Cu") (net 11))
 (segment (start 173.8325 99.8155) (end 172.1435 99.8155) (width 0.381) (layer "F.Cu") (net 11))
 (segment (start 171.5185 99.1905) (end 168.179 99.1905) (width 0.381) (layer "F.Cu") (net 11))
 (segment (start 171.5185 101.0905) (end 168.433 101.0905) (width 0.508) (layer "F.Cu") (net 14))
 (segment (start 168.433 101.0905) (end 168.113 101.4105) (width 0.508) (layer "F.Cu") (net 14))
 (segment (start 162.001304 100.3975) (end 160.843 100.3975) (width 0.381) (layer "F.Cu") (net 13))
 (segment (start 163.449 104.395) (end 163.449 101.845196) (width 0.381) (layer "F.Cu") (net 13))
 (segment (start 163.449 101.845196) (end 162.001304 100.3975) (width 0.381) (layer "F.Cu") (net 13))
 (segment (start 162.001304 100.3975) (end 162.001304 99.530196) (width 0.381) (layer "F.Cu") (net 13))
 (segment (start 162.001304 99.530196) (end 162.5365 98.995) (width 0.381) (layer "F.Cu") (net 13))
 (segment (start 159.893 98.101) (end 160.269 97.725) (width 0.508) (layer "F.Cu") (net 4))
 (segment (start 160.269 95.815) (end 160.147 95.693) (width 0.508) (layer "F.Cu") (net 4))
 (segment (start 160.269 97.725) (end 160.269 95.815) (width 0.508) (layer "F.Cu") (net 4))
 (segment (start 159.893 100.3975) (end 159.893 98.101) (width 0.508) (layer "F.Cu") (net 4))
 (segment (start 162.5365 102.551) (end 160.9645 102.551) (width 0.381) (layer "F.Cu") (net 3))
 (segment (start 161.417 103.2465) (end 160.843 102.6725) (width 0.381) (layer "F.Cu") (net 3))
 (segment (start 161.417 104.395) (end 161.417 103.2465) (width 0.381) (layer "F.Cu") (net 3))
 (segment (start 160.9645 102.551) (end 160.843 102.6725) (width 0.381) (layer "F.Cu") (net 3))
 (segment (start 158.943 102.6725) (end 158.943 105.025) (width 0.381) (layer "F.Cu") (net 16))
 (segment (start 158.943 105.025) (end 157.988 105.98) (width 0.381) (layer "F.Cu") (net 16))
 (segment (start 157.988 105.98) (end 157.988 108.458) (width 0.381) (layer "F.Cu") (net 16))
 (segment (start 168.656 113.408) (end 157.988 113.408) (width 1.27) (layer "F.Cu") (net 9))
 (segment (start 159.893 104.837) (end 159.893 102.6725) (width 0.381) (layer "F.Cu") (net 8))
 (segment (start 164.1515 105.2855) (end 160.3415 105.2855) (width 0.381) (layer "F.Cu") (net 8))
 (segment (start 164.846 105.98) (end 164.1515 105.2855) (width 0.381) (layer "F.Cu") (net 8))
 (segment (start 160.3415 105.2855) (end 159.893 104.837) (width 0.381) (layer "F.Cu") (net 8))
 (segment (start 164.846 108.458) (end 164.846 105.98) (width 0.381) (layer "F.Cu") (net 8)))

